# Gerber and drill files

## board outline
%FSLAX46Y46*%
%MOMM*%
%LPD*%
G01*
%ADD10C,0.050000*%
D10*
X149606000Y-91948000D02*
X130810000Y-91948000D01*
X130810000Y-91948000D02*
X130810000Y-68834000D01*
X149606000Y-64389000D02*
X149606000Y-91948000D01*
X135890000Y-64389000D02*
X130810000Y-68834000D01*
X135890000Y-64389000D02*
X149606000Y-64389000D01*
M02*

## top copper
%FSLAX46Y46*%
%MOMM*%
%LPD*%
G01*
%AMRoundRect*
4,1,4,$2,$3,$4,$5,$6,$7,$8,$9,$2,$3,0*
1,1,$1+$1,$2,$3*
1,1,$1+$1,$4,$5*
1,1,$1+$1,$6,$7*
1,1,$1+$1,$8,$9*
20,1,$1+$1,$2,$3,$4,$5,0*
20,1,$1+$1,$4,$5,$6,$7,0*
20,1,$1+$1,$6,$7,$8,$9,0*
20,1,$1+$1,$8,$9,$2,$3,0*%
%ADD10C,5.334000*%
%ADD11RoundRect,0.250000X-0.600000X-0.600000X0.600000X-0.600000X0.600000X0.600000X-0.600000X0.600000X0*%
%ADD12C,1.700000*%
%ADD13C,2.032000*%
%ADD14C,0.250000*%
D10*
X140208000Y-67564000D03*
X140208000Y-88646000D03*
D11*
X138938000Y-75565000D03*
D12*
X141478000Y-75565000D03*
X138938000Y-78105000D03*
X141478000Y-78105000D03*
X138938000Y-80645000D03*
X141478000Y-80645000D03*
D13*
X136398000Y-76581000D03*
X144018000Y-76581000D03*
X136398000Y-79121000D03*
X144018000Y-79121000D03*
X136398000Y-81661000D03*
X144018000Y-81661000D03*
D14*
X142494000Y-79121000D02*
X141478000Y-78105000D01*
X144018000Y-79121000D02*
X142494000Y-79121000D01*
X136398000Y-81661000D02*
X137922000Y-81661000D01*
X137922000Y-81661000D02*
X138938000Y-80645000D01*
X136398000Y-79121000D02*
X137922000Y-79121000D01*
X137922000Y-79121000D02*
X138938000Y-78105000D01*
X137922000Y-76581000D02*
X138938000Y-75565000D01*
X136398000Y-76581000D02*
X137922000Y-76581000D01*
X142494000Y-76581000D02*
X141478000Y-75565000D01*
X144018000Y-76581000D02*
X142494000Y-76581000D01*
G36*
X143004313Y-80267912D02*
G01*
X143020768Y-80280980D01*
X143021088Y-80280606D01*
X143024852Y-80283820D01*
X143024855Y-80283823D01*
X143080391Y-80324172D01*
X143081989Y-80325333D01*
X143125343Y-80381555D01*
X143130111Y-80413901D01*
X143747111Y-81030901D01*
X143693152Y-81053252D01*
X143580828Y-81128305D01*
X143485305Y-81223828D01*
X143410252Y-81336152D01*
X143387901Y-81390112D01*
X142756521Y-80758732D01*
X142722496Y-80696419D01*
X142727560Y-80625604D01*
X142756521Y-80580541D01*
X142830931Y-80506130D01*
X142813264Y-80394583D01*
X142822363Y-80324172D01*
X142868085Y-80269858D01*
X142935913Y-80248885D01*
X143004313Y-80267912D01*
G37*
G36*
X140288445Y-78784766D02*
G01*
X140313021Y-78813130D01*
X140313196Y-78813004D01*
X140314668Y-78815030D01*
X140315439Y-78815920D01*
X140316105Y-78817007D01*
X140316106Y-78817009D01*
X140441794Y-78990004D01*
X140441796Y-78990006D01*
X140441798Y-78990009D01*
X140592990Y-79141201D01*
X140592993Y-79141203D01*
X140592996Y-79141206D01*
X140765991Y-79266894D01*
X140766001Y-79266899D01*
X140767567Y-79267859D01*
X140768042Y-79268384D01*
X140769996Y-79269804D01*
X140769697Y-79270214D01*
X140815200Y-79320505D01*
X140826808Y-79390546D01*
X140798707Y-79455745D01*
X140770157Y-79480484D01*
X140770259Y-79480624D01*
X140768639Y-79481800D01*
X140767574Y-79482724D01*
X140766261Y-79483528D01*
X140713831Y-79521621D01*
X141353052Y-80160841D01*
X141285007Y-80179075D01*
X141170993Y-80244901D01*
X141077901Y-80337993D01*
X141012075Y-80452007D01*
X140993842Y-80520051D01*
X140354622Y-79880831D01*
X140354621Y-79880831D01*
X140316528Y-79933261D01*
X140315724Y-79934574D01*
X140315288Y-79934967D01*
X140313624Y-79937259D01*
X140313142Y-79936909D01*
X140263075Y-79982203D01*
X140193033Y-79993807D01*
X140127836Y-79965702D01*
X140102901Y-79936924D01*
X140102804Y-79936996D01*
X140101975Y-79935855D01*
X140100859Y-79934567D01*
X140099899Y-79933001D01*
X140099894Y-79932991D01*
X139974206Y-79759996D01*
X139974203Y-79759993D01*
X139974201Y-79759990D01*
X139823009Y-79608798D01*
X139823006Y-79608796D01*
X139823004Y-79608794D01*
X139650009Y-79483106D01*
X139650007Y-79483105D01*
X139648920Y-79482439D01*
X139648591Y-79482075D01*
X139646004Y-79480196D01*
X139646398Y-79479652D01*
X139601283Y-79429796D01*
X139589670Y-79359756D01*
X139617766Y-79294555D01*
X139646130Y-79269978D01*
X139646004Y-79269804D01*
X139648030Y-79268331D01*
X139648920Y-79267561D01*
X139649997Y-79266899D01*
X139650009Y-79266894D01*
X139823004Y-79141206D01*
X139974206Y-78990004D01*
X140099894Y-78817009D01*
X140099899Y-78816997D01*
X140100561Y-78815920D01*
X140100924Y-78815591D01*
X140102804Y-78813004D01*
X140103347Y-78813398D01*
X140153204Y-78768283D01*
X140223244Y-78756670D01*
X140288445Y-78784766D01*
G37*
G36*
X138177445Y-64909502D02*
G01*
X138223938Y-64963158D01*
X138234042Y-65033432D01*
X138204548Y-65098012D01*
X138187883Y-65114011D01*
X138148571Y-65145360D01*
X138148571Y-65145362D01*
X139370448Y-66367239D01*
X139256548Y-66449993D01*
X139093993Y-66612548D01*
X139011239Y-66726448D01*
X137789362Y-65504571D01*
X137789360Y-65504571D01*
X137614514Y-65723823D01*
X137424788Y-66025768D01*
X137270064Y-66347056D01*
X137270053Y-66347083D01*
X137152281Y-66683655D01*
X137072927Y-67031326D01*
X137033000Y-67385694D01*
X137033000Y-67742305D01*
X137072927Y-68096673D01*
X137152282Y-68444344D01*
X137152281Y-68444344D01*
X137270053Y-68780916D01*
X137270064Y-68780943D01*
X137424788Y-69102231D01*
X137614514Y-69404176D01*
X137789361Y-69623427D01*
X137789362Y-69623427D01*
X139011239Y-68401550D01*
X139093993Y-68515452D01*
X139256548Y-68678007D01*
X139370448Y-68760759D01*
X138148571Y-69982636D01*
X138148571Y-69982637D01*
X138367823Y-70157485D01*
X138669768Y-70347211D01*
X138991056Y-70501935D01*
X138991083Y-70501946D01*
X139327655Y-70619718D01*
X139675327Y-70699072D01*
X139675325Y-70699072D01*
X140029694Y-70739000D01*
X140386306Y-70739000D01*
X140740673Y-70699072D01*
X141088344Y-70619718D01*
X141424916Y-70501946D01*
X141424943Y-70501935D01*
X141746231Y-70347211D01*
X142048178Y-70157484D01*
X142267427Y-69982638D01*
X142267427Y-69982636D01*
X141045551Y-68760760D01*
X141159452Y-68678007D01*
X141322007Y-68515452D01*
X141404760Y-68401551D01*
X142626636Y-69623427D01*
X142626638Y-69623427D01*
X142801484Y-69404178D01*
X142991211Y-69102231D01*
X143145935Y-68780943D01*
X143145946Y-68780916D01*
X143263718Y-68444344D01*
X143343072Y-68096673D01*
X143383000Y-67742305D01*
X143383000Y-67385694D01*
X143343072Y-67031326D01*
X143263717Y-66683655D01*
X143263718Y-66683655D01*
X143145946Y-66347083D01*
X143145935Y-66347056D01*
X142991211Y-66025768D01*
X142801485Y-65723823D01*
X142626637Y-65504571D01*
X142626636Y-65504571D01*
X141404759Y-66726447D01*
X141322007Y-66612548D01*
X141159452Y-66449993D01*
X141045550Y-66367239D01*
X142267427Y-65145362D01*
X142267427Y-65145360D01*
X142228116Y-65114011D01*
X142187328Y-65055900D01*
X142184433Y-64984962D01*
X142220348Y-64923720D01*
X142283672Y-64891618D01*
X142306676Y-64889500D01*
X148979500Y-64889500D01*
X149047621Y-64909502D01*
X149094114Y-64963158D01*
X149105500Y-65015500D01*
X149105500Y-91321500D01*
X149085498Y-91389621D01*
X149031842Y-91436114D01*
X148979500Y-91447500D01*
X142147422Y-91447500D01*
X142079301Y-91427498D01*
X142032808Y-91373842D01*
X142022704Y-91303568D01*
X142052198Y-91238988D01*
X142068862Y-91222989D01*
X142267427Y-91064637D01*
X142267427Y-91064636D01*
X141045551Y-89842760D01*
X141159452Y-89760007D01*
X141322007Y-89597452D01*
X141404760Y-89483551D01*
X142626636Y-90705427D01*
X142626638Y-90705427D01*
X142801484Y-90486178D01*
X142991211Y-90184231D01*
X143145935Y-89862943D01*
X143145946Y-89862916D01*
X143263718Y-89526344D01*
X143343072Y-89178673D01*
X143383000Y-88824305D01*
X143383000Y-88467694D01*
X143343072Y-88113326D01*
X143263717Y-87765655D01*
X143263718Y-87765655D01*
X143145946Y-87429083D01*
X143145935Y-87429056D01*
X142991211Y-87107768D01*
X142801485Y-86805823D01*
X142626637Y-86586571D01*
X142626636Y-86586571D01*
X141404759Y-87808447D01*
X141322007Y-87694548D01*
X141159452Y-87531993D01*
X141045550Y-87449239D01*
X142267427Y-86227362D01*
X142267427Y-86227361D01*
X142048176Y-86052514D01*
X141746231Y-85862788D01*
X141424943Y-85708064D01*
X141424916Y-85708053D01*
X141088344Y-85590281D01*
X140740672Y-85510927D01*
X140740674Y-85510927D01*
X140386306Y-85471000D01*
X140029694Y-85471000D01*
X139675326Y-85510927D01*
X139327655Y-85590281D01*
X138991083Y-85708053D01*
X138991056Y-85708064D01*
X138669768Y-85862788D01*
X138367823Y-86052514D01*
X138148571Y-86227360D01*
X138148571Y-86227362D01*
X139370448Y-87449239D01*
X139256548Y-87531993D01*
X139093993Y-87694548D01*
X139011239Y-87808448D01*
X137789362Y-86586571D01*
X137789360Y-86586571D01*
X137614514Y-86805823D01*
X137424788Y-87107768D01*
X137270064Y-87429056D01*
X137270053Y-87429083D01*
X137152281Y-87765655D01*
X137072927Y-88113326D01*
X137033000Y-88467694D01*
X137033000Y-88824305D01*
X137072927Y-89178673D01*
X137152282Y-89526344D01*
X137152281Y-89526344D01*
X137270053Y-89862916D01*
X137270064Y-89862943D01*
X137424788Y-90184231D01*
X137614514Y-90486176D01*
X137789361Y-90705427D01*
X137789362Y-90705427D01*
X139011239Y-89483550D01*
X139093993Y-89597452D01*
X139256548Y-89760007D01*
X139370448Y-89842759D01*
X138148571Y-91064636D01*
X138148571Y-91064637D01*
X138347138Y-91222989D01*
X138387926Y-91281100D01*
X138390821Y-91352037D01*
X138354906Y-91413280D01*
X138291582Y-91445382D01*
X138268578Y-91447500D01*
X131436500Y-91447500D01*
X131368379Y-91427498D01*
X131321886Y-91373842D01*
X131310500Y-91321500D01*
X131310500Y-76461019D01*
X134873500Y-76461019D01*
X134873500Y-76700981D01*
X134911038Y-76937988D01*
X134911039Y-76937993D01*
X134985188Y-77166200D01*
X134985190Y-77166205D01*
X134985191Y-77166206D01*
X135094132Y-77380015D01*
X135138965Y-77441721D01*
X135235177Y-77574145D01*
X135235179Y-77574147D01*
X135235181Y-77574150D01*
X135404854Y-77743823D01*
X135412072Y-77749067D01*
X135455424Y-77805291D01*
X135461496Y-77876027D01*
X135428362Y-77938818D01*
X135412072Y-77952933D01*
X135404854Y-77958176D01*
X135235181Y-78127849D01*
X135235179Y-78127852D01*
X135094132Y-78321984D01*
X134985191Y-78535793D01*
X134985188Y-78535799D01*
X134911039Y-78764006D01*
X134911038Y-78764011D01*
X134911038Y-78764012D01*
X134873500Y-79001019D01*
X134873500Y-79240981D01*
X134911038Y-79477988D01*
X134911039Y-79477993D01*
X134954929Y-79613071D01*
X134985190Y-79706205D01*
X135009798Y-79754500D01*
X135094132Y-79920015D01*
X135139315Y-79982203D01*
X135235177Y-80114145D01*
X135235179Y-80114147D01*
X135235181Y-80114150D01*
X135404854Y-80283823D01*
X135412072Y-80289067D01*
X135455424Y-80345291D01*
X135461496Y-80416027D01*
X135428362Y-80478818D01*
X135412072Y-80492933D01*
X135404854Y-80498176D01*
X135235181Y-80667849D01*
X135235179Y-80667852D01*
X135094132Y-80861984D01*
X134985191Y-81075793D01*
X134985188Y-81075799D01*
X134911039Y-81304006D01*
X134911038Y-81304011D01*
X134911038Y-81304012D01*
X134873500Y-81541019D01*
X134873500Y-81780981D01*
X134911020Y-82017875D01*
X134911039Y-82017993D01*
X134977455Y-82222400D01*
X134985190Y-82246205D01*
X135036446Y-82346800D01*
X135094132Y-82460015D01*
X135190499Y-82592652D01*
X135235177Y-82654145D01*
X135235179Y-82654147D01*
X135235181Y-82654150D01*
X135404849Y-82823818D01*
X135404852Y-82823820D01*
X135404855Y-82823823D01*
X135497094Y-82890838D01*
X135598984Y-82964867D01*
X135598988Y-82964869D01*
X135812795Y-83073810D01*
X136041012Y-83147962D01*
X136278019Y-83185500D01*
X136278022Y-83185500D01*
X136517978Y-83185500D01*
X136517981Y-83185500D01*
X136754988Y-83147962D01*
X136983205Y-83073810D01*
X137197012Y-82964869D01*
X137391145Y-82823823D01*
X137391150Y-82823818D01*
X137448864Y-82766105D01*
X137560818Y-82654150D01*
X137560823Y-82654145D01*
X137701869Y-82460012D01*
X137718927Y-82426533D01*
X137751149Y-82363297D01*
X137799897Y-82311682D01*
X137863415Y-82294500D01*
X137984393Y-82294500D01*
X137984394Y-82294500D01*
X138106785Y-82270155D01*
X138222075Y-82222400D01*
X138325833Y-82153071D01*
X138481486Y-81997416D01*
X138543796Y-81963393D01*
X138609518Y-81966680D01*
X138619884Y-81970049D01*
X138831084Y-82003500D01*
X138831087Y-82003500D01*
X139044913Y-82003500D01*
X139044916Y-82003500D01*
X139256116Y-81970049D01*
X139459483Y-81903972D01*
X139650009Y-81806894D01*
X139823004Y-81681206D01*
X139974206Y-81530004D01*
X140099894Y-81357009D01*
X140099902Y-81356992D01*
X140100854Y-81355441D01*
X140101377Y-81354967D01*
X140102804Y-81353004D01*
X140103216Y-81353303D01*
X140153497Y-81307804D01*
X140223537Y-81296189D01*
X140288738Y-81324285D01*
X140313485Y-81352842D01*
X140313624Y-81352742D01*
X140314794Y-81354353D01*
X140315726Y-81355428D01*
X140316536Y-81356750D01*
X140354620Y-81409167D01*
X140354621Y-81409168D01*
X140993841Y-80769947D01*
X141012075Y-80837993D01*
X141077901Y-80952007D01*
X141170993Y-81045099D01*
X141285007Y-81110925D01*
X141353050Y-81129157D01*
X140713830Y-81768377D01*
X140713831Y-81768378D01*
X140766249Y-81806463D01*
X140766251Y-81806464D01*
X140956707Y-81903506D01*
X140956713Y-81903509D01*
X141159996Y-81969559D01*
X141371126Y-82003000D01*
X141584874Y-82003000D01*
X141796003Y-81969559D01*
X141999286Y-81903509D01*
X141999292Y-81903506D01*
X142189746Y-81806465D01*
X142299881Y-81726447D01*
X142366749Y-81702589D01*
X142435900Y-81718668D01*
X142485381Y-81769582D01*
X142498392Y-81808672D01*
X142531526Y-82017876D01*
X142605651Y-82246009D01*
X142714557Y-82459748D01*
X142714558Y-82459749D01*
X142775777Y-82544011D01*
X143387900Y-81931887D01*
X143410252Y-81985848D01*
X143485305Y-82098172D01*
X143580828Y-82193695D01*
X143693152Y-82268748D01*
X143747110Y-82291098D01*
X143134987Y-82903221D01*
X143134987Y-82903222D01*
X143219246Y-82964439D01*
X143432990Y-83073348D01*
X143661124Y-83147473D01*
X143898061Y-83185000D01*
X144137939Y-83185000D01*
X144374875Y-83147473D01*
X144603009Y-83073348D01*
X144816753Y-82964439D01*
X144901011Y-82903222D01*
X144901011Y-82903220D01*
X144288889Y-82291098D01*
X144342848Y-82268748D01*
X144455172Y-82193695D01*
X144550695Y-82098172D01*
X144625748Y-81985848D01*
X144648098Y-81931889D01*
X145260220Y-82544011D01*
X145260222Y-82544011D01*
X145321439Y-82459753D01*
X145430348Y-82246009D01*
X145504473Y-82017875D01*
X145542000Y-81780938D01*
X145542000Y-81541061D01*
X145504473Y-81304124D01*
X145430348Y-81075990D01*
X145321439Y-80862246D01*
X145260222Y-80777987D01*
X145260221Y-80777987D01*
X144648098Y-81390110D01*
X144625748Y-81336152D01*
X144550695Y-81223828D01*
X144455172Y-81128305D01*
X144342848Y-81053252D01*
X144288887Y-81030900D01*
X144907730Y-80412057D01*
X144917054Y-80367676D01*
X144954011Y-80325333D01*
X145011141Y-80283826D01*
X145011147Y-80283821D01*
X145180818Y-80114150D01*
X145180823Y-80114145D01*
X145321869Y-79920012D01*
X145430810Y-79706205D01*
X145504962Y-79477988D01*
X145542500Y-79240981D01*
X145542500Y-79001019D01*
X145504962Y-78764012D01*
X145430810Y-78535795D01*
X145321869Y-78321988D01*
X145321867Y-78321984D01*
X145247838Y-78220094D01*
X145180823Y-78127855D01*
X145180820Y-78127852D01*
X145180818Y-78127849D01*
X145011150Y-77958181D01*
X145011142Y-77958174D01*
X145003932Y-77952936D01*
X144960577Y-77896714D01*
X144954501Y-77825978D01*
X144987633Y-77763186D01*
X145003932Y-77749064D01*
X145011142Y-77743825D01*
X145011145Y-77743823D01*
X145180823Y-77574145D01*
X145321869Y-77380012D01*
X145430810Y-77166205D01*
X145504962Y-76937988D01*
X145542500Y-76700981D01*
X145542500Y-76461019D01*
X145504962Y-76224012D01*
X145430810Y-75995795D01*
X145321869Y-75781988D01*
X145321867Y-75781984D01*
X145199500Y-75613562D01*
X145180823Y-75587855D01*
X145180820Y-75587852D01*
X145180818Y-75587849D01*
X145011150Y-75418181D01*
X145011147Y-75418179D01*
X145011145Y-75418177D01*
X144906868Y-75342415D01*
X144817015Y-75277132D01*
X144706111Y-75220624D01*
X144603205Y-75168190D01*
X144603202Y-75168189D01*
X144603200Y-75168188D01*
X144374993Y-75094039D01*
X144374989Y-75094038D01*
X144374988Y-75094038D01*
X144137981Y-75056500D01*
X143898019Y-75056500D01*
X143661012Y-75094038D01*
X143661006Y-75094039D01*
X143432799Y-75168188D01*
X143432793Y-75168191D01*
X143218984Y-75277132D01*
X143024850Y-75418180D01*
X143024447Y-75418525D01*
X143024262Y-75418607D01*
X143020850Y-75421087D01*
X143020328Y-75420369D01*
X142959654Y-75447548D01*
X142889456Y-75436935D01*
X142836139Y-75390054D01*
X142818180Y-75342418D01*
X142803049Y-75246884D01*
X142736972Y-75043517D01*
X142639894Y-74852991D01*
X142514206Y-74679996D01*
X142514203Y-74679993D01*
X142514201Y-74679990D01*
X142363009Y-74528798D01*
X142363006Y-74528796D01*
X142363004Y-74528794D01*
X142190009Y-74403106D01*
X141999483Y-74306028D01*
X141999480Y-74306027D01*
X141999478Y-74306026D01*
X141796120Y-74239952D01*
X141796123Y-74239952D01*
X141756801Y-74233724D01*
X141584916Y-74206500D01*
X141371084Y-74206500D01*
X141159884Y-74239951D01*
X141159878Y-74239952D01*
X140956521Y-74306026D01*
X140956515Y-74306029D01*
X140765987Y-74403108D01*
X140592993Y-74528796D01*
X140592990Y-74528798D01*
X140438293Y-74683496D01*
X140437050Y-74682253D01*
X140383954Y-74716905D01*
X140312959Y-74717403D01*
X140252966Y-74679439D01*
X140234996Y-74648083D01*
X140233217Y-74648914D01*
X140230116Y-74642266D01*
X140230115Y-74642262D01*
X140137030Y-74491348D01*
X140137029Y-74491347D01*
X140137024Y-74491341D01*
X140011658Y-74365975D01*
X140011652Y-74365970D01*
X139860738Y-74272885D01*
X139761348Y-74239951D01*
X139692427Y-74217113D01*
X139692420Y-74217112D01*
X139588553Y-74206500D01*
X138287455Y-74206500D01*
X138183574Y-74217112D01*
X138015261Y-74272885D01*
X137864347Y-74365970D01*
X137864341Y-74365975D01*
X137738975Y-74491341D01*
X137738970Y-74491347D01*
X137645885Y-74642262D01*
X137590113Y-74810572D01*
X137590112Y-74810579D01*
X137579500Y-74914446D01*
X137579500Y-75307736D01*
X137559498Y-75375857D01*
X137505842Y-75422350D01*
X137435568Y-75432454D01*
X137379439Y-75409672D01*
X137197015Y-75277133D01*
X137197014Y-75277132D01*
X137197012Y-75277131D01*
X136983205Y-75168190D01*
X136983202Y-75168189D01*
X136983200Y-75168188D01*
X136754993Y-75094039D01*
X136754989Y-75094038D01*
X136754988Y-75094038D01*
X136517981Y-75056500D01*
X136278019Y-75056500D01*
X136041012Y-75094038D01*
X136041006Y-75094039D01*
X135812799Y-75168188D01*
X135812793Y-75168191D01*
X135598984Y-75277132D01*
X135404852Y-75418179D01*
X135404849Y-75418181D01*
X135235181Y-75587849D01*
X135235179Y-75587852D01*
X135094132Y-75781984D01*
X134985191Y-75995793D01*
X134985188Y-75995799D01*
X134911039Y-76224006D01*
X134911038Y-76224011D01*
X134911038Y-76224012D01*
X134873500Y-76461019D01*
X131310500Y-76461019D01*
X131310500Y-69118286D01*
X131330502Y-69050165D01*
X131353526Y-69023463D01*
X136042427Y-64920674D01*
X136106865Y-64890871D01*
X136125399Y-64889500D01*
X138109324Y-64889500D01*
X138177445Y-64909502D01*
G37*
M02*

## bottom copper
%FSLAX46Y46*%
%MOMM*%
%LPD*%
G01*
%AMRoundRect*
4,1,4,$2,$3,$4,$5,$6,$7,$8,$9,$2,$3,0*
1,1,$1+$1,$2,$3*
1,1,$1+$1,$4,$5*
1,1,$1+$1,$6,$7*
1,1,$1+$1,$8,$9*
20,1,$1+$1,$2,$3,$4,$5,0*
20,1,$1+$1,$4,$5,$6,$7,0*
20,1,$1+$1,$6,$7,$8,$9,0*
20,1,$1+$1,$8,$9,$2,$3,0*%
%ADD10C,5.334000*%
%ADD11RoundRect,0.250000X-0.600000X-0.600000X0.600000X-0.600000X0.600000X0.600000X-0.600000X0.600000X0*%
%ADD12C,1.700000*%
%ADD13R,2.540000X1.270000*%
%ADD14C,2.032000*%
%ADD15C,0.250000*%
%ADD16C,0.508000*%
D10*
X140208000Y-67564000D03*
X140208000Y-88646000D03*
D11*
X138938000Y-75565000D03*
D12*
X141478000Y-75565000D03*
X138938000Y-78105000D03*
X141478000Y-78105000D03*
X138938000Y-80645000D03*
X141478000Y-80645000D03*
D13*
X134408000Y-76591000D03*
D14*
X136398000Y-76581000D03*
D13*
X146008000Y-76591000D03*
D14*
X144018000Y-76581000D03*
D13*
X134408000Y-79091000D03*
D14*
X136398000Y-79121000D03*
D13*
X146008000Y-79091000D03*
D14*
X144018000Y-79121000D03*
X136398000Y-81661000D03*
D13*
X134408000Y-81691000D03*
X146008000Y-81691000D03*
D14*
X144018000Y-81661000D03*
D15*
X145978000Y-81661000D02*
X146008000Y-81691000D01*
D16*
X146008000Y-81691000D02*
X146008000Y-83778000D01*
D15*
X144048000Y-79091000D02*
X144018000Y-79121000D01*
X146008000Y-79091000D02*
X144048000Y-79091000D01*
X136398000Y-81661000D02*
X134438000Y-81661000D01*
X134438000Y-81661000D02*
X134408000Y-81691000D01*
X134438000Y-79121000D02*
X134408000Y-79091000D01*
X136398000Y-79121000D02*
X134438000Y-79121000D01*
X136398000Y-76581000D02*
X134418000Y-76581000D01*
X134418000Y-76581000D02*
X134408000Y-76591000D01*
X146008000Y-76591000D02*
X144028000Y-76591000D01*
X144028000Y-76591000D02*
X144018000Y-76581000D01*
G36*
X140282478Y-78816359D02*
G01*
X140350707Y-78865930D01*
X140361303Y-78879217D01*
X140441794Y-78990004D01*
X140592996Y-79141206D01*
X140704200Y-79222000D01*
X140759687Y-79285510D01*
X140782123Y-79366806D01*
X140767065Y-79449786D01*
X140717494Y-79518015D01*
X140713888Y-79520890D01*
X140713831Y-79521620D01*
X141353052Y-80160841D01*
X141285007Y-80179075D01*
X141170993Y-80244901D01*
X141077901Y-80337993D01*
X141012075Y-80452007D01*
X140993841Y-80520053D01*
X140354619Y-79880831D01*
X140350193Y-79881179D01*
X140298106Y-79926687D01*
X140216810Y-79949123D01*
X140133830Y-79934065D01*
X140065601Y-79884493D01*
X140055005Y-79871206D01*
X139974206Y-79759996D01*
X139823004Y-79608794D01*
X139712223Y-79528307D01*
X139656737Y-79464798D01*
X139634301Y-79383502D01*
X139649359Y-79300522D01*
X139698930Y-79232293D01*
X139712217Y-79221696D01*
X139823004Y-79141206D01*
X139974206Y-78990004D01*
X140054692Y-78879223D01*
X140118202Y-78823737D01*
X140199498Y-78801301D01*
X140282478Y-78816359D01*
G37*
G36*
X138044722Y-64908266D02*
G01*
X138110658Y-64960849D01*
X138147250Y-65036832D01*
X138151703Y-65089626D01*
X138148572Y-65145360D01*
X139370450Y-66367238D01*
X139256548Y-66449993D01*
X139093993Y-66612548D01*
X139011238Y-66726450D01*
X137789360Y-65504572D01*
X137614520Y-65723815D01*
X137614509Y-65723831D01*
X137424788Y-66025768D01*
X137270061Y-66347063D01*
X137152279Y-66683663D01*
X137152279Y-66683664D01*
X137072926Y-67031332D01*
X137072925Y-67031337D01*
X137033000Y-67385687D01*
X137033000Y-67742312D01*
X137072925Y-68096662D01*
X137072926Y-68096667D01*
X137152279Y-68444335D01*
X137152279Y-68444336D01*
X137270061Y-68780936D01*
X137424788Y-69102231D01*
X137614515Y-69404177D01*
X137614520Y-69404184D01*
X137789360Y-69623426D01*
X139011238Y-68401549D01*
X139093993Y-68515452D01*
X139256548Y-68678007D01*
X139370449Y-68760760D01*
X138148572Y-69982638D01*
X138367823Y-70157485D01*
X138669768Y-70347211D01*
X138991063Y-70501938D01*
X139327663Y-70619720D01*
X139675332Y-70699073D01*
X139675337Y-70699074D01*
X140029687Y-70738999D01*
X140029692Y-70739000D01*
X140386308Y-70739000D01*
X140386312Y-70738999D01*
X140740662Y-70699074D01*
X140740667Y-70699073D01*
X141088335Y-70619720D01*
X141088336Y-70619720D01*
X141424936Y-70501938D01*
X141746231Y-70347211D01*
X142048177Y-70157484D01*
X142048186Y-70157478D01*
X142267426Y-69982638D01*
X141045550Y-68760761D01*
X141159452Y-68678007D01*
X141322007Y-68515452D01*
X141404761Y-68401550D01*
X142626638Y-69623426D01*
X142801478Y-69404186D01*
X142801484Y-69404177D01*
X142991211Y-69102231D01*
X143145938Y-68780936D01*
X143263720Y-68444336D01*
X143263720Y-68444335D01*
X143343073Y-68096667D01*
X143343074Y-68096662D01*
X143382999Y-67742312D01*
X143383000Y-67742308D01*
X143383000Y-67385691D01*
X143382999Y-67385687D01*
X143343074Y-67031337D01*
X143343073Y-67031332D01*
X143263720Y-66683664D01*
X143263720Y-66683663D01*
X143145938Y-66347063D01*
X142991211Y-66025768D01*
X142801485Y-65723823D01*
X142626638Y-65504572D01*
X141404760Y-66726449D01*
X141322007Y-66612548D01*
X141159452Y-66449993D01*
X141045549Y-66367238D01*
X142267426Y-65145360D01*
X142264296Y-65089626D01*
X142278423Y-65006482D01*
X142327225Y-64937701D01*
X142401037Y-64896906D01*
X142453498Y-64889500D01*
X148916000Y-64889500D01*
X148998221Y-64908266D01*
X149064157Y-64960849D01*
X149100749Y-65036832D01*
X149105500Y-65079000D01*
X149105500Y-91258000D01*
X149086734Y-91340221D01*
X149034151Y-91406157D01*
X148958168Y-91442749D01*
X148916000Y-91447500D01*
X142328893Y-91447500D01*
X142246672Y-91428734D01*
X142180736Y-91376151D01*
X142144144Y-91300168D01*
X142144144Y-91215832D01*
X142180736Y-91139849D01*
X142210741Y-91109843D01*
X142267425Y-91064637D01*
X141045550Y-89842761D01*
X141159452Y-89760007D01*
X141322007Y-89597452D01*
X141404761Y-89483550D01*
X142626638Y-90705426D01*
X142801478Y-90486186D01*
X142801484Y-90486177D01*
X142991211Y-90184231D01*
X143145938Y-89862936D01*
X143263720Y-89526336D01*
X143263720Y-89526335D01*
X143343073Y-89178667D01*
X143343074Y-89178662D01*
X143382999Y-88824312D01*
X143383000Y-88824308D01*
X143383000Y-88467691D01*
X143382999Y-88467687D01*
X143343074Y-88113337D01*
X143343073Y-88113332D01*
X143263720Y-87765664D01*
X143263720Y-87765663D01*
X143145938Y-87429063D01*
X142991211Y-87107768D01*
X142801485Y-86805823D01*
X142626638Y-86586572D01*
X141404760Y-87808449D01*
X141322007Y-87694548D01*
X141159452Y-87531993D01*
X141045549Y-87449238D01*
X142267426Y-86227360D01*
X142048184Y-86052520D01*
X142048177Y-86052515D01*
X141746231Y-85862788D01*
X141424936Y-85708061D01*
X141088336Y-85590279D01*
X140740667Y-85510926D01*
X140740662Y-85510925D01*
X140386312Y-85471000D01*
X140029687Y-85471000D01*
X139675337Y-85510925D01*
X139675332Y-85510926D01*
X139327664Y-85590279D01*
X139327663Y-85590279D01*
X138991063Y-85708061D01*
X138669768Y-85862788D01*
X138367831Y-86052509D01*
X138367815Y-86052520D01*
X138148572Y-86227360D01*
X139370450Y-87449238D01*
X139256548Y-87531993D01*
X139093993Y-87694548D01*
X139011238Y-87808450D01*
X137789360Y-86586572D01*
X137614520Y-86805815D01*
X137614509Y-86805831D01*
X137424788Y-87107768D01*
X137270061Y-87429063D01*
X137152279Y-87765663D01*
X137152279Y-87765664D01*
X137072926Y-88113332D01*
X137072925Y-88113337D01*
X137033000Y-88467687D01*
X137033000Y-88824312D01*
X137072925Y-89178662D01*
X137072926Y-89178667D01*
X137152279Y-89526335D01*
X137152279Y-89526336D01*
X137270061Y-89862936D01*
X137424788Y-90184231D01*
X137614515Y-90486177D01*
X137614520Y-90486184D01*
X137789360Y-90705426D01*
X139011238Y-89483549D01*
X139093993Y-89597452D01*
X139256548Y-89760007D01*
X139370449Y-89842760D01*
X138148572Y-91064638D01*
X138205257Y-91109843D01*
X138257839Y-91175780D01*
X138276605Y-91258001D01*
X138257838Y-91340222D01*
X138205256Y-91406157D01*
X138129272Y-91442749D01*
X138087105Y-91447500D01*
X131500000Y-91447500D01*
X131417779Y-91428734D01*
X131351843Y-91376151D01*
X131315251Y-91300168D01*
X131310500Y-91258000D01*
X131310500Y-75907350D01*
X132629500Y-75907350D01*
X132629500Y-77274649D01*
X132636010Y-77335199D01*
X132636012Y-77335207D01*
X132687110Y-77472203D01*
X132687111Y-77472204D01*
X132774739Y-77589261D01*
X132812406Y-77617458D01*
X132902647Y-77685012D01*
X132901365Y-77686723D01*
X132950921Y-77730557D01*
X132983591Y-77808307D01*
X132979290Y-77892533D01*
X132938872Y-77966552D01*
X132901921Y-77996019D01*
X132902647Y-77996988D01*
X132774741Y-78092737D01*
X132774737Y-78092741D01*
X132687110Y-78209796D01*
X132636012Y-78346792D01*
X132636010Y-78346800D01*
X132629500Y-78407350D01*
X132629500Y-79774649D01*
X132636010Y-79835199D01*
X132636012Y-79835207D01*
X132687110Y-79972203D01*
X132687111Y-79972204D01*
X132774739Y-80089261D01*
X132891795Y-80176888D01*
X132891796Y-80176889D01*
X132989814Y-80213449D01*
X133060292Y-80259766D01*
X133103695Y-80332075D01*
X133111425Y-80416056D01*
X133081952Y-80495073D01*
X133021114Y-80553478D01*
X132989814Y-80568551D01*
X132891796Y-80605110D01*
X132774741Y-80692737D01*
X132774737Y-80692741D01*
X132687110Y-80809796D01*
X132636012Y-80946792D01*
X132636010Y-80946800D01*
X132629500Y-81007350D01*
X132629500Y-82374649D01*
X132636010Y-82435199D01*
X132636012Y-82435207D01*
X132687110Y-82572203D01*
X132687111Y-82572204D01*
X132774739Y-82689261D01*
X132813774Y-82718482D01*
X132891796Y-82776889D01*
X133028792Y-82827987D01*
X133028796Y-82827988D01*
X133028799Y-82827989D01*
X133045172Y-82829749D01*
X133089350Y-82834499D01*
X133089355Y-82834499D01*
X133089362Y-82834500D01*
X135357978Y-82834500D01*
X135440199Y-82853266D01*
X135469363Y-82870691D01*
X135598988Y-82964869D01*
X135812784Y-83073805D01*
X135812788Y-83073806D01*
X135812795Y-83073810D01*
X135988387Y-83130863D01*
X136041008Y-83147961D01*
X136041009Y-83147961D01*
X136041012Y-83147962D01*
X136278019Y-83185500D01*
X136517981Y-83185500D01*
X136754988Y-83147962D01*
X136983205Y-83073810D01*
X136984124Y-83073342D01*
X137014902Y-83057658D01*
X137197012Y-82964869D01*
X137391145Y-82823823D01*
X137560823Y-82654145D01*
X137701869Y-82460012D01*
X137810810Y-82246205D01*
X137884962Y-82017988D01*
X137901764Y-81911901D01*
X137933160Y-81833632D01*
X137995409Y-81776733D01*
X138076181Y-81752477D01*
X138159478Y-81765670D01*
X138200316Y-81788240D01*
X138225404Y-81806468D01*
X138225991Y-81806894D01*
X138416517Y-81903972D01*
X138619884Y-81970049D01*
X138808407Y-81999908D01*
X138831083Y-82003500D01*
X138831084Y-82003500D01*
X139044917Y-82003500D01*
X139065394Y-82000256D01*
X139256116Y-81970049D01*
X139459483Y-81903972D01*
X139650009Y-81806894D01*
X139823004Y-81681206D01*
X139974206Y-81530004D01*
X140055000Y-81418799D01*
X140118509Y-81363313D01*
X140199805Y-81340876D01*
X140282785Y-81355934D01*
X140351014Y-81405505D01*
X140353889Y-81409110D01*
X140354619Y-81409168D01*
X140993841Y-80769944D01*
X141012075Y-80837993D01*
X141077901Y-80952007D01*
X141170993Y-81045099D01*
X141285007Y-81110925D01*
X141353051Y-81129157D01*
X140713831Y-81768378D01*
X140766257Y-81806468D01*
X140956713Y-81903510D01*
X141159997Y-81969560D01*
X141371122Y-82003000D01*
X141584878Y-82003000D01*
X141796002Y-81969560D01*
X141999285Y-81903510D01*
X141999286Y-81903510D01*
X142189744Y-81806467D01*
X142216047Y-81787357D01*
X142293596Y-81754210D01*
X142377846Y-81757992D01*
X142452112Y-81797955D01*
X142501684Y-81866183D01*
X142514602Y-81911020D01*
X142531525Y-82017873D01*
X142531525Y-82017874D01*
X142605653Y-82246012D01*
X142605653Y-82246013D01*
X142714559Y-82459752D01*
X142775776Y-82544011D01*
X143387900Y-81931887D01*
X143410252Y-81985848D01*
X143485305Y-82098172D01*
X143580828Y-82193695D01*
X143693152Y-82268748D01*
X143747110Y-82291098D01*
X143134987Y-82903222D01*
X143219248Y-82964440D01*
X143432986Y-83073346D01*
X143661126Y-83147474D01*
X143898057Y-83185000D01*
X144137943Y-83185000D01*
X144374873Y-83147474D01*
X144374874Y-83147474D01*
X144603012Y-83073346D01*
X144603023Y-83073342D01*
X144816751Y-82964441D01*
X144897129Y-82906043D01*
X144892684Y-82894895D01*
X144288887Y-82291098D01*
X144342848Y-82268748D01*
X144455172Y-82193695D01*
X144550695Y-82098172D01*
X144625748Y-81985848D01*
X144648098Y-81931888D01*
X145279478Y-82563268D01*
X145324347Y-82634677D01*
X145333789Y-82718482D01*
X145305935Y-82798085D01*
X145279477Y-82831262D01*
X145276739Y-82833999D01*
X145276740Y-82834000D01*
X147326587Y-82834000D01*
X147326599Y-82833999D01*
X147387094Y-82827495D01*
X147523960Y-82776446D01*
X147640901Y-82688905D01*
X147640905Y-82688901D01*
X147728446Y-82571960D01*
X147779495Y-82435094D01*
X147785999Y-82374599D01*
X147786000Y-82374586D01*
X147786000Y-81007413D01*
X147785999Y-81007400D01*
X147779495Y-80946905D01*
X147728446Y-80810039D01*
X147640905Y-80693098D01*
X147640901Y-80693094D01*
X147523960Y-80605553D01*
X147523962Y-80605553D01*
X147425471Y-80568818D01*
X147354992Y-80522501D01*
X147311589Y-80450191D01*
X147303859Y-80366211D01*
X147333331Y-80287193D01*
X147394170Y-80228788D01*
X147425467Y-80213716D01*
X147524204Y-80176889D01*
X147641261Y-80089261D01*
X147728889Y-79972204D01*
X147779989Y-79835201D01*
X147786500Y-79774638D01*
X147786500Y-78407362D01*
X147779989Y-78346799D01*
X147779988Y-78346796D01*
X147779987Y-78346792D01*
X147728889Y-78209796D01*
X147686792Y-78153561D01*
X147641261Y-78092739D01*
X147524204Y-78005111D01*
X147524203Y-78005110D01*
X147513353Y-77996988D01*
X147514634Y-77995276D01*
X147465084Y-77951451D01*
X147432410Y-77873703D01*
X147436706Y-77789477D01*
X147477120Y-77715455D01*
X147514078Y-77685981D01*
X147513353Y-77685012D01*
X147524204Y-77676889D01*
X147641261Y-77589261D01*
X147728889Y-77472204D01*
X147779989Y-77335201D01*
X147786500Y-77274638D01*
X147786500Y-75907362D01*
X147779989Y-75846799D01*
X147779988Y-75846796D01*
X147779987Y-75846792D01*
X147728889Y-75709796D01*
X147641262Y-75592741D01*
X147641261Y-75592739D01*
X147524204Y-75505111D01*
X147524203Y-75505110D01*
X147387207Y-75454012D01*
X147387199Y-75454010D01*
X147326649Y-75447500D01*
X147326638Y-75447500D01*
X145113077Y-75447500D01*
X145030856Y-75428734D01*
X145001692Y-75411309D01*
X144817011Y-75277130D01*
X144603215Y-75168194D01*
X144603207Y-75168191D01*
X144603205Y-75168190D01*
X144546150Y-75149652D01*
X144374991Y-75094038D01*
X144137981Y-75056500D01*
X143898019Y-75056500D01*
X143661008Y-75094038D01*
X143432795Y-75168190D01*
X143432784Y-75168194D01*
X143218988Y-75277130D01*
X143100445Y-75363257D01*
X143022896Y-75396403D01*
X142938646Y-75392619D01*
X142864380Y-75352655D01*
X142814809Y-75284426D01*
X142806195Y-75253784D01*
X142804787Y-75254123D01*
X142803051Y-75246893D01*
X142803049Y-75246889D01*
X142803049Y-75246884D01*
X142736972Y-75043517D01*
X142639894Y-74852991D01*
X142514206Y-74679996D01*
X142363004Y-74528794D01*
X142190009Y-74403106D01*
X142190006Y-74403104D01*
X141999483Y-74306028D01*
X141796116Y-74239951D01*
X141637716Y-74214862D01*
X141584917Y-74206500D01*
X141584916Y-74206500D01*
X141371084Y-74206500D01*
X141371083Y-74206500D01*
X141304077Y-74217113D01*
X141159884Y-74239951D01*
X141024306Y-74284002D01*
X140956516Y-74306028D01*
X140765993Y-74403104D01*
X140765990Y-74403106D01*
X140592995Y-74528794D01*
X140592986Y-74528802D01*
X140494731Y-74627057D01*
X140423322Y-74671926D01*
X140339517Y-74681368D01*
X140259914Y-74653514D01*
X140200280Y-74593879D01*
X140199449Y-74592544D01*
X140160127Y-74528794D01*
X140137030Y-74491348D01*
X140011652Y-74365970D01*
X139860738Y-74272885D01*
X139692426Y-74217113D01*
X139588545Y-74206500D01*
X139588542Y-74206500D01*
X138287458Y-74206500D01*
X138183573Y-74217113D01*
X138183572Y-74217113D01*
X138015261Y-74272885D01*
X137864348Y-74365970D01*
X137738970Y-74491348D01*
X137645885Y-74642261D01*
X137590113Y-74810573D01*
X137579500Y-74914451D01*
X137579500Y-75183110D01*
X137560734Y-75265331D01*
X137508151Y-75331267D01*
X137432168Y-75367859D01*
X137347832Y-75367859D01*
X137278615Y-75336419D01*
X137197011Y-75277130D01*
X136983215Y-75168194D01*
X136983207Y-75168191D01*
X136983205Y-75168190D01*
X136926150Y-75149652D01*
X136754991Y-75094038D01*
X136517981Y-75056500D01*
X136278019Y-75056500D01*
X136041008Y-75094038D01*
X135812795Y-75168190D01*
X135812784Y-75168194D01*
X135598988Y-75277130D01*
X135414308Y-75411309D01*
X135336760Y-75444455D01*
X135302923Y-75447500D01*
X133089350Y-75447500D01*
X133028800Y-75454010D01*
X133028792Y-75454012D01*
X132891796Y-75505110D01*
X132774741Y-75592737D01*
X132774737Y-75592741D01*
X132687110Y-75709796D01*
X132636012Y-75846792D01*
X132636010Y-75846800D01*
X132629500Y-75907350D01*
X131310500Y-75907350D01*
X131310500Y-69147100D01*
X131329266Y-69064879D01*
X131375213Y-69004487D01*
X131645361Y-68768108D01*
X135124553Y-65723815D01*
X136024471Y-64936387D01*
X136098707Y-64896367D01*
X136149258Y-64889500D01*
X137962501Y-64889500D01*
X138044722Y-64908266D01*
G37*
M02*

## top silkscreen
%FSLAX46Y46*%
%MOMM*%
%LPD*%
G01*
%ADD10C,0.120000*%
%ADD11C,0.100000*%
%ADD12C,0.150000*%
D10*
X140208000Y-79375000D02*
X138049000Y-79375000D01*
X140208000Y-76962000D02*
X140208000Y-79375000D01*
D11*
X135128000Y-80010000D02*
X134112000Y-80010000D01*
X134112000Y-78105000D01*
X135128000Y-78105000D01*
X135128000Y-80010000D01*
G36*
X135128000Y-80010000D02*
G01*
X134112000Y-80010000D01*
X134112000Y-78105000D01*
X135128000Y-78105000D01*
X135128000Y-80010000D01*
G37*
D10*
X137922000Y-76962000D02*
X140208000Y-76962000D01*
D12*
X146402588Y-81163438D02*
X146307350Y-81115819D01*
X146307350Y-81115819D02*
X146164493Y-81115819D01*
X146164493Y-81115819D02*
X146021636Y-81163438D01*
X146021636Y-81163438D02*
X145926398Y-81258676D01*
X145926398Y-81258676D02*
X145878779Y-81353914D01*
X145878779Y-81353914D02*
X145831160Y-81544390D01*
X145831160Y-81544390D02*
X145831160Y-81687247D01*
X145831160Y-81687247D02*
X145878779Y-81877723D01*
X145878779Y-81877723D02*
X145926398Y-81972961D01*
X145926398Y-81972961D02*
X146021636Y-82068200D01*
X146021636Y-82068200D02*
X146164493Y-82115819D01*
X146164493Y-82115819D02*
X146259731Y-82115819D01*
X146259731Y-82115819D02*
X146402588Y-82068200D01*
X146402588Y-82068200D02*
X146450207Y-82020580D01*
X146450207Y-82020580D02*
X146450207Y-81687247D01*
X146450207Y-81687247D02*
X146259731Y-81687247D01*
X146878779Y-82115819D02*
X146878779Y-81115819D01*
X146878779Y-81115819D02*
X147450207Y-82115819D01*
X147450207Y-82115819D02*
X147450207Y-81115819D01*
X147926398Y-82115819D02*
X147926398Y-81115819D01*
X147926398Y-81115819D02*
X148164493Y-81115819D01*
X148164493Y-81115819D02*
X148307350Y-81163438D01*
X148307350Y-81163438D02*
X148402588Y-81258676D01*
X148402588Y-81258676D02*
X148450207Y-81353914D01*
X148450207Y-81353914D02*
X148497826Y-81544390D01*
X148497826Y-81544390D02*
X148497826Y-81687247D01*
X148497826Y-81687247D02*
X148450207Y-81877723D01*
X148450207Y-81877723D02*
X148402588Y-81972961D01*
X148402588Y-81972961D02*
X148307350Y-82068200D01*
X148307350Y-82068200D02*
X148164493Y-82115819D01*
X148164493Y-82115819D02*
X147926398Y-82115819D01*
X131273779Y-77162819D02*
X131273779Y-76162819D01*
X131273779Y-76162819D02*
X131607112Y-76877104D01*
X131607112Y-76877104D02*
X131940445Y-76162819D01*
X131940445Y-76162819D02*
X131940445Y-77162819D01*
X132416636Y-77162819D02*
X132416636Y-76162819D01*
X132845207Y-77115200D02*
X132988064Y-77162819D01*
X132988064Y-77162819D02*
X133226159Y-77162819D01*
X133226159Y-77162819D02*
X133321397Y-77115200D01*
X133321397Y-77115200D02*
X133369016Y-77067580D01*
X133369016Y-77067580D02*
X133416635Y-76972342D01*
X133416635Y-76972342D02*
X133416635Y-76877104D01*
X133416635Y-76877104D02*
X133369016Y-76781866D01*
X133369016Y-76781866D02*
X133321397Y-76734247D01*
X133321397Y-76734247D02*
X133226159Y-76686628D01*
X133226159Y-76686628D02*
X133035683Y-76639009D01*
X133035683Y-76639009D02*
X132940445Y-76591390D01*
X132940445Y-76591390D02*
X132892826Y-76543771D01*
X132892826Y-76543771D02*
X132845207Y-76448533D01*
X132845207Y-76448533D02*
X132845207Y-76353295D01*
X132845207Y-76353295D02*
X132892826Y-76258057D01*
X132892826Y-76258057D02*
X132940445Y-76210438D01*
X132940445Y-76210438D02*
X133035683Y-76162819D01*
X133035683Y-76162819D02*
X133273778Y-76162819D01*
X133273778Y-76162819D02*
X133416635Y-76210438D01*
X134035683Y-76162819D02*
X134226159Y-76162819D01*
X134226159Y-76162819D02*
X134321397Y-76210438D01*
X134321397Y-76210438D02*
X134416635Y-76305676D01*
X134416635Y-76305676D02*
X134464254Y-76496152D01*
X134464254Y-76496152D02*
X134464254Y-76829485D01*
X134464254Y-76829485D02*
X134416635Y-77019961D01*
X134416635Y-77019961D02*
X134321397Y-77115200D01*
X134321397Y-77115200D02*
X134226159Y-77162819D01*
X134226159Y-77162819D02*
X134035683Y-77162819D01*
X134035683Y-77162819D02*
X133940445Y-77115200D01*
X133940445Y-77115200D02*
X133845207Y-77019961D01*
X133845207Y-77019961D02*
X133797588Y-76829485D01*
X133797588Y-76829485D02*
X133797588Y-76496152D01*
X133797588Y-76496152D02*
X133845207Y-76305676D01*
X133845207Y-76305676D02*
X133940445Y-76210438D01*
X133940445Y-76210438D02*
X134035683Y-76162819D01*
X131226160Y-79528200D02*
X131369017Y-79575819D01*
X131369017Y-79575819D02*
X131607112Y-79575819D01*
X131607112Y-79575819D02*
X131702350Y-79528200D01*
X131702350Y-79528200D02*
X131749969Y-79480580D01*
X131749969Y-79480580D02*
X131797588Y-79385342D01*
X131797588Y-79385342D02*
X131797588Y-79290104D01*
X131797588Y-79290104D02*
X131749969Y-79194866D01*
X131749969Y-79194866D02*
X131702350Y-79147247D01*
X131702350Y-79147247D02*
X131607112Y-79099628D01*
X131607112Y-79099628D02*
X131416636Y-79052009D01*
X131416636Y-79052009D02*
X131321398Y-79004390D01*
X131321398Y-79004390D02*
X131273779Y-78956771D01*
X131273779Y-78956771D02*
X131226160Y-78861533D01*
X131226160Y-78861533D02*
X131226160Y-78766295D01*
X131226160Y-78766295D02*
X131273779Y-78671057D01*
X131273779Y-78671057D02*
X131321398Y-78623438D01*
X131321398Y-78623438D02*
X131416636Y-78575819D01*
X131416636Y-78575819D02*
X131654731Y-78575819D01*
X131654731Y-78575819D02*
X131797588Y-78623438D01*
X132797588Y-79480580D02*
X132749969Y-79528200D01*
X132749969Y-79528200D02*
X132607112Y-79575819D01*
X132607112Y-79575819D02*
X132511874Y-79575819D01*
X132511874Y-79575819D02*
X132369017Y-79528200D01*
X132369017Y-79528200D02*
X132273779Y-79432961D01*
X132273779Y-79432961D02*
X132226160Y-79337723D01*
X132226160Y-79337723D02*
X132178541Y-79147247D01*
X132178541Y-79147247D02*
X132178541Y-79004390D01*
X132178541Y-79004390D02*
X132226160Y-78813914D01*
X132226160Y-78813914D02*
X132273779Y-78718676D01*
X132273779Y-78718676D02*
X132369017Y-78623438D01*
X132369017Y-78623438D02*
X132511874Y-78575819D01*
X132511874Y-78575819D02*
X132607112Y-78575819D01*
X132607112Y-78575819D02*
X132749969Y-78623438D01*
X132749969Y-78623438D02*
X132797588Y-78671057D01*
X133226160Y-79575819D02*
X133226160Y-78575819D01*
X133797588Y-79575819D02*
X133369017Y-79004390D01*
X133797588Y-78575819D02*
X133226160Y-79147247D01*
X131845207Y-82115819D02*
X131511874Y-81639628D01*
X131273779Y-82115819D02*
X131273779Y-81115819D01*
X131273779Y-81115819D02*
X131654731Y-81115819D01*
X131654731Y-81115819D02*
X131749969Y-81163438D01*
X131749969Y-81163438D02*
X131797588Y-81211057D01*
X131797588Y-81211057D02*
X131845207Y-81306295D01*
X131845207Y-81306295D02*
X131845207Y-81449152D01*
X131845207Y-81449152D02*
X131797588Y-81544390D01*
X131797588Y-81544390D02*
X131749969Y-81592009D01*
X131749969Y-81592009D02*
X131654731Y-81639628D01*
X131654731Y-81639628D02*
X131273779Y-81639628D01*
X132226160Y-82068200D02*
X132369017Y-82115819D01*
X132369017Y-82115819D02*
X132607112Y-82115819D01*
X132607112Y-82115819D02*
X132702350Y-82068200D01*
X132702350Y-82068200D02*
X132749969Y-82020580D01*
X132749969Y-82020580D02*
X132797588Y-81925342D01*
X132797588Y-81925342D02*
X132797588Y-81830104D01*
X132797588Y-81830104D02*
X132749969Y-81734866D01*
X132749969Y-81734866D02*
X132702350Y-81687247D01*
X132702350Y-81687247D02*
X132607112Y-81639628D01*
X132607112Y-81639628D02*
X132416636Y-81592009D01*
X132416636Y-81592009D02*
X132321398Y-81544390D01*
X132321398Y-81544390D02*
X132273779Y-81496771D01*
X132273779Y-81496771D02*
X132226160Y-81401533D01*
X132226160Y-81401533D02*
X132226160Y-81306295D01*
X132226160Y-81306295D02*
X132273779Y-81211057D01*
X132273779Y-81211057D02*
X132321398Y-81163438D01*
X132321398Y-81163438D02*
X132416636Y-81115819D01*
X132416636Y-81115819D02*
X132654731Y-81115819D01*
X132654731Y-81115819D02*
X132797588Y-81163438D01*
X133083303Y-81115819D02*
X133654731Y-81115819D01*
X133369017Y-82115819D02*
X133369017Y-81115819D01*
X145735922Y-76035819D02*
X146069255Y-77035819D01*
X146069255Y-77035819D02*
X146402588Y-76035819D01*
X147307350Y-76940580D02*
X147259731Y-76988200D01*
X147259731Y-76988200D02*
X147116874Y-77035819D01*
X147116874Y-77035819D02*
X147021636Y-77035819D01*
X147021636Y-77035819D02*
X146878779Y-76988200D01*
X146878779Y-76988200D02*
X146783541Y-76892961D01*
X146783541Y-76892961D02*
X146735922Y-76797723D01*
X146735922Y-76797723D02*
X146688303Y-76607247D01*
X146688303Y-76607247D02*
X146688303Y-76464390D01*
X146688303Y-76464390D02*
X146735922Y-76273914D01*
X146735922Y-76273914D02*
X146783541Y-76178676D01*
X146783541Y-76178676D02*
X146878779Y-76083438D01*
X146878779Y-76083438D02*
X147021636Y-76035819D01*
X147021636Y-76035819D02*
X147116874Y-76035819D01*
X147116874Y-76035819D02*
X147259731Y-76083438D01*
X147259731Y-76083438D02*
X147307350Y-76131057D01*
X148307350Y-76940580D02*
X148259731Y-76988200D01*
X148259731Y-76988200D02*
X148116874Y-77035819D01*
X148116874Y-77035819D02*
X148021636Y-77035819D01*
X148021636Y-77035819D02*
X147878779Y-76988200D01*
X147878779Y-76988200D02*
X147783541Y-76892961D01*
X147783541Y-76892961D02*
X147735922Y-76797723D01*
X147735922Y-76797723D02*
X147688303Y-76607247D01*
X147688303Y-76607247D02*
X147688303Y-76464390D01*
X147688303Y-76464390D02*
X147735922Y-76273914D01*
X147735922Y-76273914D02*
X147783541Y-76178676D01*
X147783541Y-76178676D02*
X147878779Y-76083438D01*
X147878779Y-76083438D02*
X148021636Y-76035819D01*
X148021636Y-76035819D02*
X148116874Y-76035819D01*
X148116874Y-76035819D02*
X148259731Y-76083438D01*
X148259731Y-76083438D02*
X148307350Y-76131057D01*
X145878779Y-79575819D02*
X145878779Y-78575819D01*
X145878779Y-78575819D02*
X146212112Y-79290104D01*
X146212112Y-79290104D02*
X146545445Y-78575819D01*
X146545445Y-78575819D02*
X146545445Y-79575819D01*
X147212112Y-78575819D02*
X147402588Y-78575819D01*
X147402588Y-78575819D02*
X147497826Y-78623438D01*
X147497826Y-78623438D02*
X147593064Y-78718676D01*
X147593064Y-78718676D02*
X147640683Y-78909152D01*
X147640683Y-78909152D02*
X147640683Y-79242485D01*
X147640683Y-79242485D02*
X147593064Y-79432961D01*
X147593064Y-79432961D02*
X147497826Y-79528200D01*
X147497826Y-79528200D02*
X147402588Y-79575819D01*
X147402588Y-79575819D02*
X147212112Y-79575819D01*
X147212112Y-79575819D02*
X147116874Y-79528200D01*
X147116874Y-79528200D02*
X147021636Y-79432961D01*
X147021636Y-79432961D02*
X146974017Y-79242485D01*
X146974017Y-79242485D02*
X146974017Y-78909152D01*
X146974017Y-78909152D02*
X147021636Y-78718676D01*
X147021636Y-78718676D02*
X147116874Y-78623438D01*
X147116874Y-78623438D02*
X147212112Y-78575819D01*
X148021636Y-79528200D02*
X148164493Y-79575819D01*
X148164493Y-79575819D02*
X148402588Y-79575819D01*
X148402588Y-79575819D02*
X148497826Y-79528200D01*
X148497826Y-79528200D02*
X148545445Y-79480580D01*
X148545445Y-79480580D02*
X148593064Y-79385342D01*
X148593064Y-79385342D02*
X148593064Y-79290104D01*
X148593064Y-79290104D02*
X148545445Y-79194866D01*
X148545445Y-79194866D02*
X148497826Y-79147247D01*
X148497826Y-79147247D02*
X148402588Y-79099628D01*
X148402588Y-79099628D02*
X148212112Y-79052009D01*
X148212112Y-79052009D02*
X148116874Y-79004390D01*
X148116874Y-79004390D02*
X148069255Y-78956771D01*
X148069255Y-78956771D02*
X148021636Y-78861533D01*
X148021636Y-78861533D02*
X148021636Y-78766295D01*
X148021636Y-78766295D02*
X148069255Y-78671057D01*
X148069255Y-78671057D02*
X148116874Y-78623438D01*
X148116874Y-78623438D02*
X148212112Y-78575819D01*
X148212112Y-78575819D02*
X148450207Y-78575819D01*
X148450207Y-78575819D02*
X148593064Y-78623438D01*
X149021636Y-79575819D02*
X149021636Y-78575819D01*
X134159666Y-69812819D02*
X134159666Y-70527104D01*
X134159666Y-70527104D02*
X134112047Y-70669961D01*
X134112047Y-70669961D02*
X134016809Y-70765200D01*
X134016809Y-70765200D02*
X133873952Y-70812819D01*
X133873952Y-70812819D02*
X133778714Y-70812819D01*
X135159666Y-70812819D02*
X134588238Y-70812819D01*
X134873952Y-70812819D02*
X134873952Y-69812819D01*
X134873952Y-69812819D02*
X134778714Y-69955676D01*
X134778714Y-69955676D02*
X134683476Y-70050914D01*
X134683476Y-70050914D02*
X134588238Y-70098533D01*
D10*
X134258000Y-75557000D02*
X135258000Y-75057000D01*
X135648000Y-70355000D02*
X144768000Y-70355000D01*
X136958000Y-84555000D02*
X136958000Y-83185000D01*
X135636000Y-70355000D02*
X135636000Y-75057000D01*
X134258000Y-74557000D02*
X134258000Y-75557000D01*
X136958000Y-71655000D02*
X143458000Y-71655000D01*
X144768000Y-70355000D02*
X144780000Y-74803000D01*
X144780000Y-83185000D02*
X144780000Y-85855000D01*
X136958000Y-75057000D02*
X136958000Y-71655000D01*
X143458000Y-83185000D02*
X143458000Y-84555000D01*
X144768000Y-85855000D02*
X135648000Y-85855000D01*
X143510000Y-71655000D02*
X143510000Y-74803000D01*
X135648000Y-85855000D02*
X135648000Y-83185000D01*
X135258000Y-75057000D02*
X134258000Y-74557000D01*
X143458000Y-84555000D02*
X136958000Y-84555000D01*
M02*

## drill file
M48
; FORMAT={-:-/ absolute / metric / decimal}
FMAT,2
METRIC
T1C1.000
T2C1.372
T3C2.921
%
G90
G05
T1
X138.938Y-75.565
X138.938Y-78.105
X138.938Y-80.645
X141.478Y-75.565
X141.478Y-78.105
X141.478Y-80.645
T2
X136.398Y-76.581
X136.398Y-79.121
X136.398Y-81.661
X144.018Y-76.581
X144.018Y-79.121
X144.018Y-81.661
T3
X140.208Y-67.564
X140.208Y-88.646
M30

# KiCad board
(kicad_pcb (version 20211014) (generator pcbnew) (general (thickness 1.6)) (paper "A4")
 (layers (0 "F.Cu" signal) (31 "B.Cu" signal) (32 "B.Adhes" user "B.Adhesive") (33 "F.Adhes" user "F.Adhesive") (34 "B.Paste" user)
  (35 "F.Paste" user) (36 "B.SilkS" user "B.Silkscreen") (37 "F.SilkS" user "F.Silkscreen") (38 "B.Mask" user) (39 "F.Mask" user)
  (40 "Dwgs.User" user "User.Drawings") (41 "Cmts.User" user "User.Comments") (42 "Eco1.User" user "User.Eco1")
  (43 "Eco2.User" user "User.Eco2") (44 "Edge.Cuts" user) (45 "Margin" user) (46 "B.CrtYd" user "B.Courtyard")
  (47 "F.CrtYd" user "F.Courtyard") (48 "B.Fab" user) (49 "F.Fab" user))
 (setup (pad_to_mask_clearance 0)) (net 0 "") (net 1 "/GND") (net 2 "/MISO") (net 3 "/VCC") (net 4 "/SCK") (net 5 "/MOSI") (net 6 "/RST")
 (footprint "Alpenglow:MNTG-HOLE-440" (layer "F.Cu") (at 140.208 66.294)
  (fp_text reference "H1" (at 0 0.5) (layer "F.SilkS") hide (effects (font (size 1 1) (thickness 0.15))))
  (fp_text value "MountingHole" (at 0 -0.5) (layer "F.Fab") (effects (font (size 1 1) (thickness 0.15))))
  (pad "1" thru_hole circle locked (at 0 1.27) (size 5.334 5.334) (drill 2.921) (layers *.Cu *.Mask) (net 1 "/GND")))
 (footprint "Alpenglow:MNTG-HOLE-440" (layer "F.Cu") (at 140.208 87.376)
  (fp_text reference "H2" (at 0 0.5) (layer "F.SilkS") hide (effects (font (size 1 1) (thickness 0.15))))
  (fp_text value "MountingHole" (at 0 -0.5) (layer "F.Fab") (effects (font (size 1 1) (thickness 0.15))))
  (pad "2" thru_hole circle locked (at 0 1.27) (size 5.334 5.334) (drill 2.921) (layers *.Cu *.Mask) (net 1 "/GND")))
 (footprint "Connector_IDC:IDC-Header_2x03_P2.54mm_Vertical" (layer "F.Cu") (at 138.938 75.565)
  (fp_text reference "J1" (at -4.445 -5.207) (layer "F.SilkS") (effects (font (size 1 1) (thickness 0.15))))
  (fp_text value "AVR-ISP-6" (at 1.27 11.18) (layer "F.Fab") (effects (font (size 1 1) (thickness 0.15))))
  (fp_line (start -4.68 -0.008) (end -3.68 -0.508) (layer "F.SilkS") (width 0.12))
  (fp_line (start -3.29 -5.21) (end 5.83 -5.21) (layer "F.SilkS") (width 0.12))
  (fp_line (start -1.98 8.99) (end -1.98 7.62) (layer "F.SilkS") (width 0.12))
  (fp_line (start -3.302 -5.21) (end -3.302 -0.508) (layer "F.SilkS") (width 0.12))
  (fp_line (start -4.68 -1.008) (end -4.68 -0.008) (layer "F.SilkS") (width 0.12))
  (fp_line (start -1.98 -3.91) (end 4.52 -3.91) (layer "F.SilkS") (width 0.12))
  (fp_line (start 5.83 -5.21) (end 5.842 -0.762) (layer "F.SilkS") (width 0.12))
  (fp_line (start 5.842 7.62) (end 5.842 10.29) (layer "F.SilkS") (width 0.12))
  (fp_line (start -1.98 -0.508) (end -1.98 -3.91) (layer "F.SilkS") (width 0.12))
  (fp_line (start 4.52 7.62) (end 4.52 8.99) (layer "F.SilkS") (width 0.12))
  (fp_line (start 5.83 10.29) (end -3.29 10.29) (layer "F.SilkS") (width 0.12))
  (fp_line (start 4.572 -3.91) (end 4.572 -0.762) (layer "F.SilkS") (width 0.12))
  (fp_line (start -3.29 10.29) (end -3.29 7.62) (layer "F.SilkS") (width 0.12))
  (fp_line (start -3.68 -0.508) (end -4.68 -1.008) (layer "F.SilkS") (width 0.12))
  (fp_line (start 4.52 8.99) (end -1.98 8.99) (layer "F.SilkS") (width 0.12))
  (pad "1" thru_hole roundrect locked (at 0 0) (size 1.7 1.7) (drill 1) (layers *.Cu *.Mask) (roundrect_rratio 0.1470588235) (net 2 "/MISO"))
  (pad "2" thru_hole circle locked (at 2.54 0) (size 1.7 1.7) (drill 1) (layers *.Cu *.Mask) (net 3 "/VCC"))
  (pad "3" thru_hole circle locked (at 0 2.54) (size 1.7 1.7) (drill 1) (layers *.Cu *.Mask) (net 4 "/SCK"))
  (pad "4" thru_hole circle locked (at 2.54 2.54) (size 1.7 1.7) (drill 1) (layers *.Cu *.Mask) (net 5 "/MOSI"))
  (pad "5" thru_hole circle locked (at 0 5.08) (size 1.7 1.7) (drill 1) (layers *.Cu *.Mask) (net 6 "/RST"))
  (pad "6" thru_hole circle locked (at 2.54 5.08) (size 1.7 1.7) (drill 1) (layers *.Cu *.Mask) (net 1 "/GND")))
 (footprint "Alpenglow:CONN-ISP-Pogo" (layer "F.Cu") (at 140.208 80.391)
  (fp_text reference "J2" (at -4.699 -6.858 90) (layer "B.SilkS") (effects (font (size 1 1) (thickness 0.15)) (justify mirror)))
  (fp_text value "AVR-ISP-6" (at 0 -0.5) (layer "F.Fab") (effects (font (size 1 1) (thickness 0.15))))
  (pad "1" smd rect locked (at -5.8 -3.8) (size 2.54 1.27) (layers "B.Cu" "B.Paste" "B.Mask") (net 2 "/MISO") (zone_connect 0))
  (pad "1" thru_hole circle locked (at -3.81 -3.81) (size 2.032 2.032) (drill 1.3716) (layers *.Cu *.Mask) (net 2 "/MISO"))
  (pad "2" smd rect locked (at 5.8 -3.8) (size 2.54 1.27) (layers "B.Cu" "B.Paste" "B.Mask") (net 3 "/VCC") (zone_connect 0))
  (pad "2" thru_hole circle locked (at 3.81 -3.81) (size 2.032 2.032) (drill 1.3716) (layers *.Cu *.Mask) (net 3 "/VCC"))
  (pad "3" smd rect locked (at -5.8 -1.3) (size 2.54 1.27) (layers "B.Cu" "B.Paste" "B.Mask") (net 4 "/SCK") (zone_connect 0))
  (pad "3" thru_hole circle locked (at -3.81 -1.27) (size 2.032 2.032) (drill 1.3716) (layers *.Cu *.Mask) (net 4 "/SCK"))
  (pad "4" smd rect locked (at 5.8 -1.3) (size 2.54 1.27) (layers "B.Cu" "B.Paste" "B.Mask") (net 5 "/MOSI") (zone_connect 0))
  (pad "4" thru_hole circle locked (at 3.81 -1.27) (size 2.032 2.032) (drill 1.3716) (layers *.Cu *.Mask) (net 5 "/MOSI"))
  (pad "5" thru_hole circle locked (at -3.81 1.27) (size 2.032 2.032) (drill 1.3716) (layers *.Cu *.Mask) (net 6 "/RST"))
  (pad "5" smd rect locked (at -5.8 1.3) (size 2.54 1.27) (layers "B.Cu" "B.Paste" "B.Mask") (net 6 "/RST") (zone_connect 0))
  (pad "6" smd rect locked (at 5.8 1.3) (size 2.54 1.27) (layers "B.Cu" "B.Paste" "B.Mask") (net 1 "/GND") (zone_connect 0))
  (pad "6" thru_hole circle locked (at 3.81 1.27) (size 2.032 2.032) (drill 1.3716) (layers *.Cu *.Mask) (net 1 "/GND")))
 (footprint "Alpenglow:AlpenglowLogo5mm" (layer "B.Cu") (at 146.685 70.485 -90)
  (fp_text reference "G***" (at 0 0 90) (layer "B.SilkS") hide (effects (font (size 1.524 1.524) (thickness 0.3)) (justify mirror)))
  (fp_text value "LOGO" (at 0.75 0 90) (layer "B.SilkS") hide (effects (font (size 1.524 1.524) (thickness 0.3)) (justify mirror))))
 (gr_line (start 140.208 79.375) (end 138.049 79.375) (layer "F.SilkS") (width 0.12))
 (gr_line (start 140.208 76.962) (end 140.208 79.375) (layer "F.SilkS") (width 0.12))
 (gr_poly (pts (xy 135.128 80.01) (xy 134.112 80.01) (xy 134.112 78.105) (xy 135.128 78.105)) (layer "F.SilkS") (width 0.1) (fill solid))
 (gr_line (start 137.922 76.962) (end 140.208 76.962) (layer "F.SilkS") (width 0.12))
 (gr_line (start 149.606 91.948) (end 130.81 91.948) (layer "Edge.Cuts") (width 0.05))
 (gr_line (start 130.81 91.948) (end 130.81 68.834) (layer "Edge.Cuts") (width 0.05))
 (gr_line (start 149.606 64.389) (end 149.606 91.948) (layer "Edge.Cuts") (width 0.05))
 (gr_line (start 135.89 64.389) (end 130.81 68.834) (layer "Edge.Cuts") (width 0.05))
 (gr_line (start 135.89 64.389) (end 149.606 64.389) (layer "Edge.Cuts") (width 0.05))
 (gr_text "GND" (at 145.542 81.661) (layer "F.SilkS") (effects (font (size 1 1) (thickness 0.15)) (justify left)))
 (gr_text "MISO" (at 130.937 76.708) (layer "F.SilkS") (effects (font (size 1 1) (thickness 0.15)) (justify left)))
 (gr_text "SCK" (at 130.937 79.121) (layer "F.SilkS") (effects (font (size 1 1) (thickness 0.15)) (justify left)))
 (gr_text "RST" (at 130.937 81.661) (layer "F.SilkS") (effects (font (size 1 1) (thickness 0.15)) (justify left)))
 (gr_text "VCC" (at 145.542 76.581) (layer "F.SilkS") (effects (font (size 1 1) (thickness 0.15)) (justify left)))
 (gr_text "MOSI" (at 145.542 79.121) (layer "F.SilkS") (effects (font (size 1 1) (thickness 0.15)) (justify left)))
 (segment (start 145.978 81.661) (end 146.008 81.691) (width 0.25) (layer "B.Cu") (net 1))
 (segment (start 146.008 81.691) (end 146.008 83.778) (width 0.508) (layer "B.Cu") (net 1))
 (segment (start 142.494 79.121) (end 141.478 78.105) (width 0.25) (layer "F.Cu") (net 5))
 (segment (start 144.018 79.121) (end 142.494 79.121) (width 0.25) (layer "F.Cu") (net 5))
 (segment (start 144.048 79.091) (end 144.018 79.121) (width 0.25) (layer "B.Cu") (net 5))
 (segment (start 146.008 79.091) (end 144.048 79.091) (width 0.25) (layer "B.Cu") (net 5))
 (segment (start 136.398 81.661) (end 137.922 81.661) (width 0.25) (layer "F.Cu") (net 6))
 (segment (start 137.922 81.661) (end 138.938 80.645) (width 0.25) (layer "F.Cu") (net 6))
 (segment (start 136.398 81.661) (end 134.438 81.661) (width 0.25) (layer "B.Cu") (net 6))
 (segment (start 134.438 81.661) (end 134.408 81.691) (width 0.25) (layer "B.Cu") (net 6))
 (segment (start 136.398 79.121) (end 137.922 79.121) (width 0.25) (layer "F.Cu") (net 4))
 (segment (start 137.922 79.121) (end 138.938 78.105) (width 0.25) (layer "F.Cu") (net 4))
 (segment (start 134.438 79.121) (end 134.408 79.091) (width 0.25) (layer "B.Cu") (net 4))
 (segment (start 136.398 79.121) (end 134.438 79.121) (width 0.25) (layer "B.Cu") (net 4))
 (segment (start 137.922 76.581) (end 138.938 75.565) (width 0.25) (layer "F.Cu") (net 2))
 (segment (start 136.398 76.581) (end 137.922 76.581) (width 0.25) (layer "F.Cu") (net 2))
 (segment (start 136.398 76.581) (end 134.418 76.581) (width 0.25) (layer "B.Cu") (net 2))
 (segment (start 134.418 76.581) (end 134.408 76.591) (width 0.25) (layer "B.Cu") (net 2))
 (segment (start 142.494 76.581) (end 141.478 75.565) (width 0.25) (layer "F.Cu") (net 3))
 (segment (start 144.018 76.581) (end 142.494 76.581) (width 0.25) (layer "F.Cu") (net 3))
 (segment (start 146.008 76.591) (end 144.028 76.591) (width 0.25) (layer "B.Cu") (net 3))
 (segment (start 144.028 76.591) (end 144.018 76.581) (width 0.25) (layer "B.Cu") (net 3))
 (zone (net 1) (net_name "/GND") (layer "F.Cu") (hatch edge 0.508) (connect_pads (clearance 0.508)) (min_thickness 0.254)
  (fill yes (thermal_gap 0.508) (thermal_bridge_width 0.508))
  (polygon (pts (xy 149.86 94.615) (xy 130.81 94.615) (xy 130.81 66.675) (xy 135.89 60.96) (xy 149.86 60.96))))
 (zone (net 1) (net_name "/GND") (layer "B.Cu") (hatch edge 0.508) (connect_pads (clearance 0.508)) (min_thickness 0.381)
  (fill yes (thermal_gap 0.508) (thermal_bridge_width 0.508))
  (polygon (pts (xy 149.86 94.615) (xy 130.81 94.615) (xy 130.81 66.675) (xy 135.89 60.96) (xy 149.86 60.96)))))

